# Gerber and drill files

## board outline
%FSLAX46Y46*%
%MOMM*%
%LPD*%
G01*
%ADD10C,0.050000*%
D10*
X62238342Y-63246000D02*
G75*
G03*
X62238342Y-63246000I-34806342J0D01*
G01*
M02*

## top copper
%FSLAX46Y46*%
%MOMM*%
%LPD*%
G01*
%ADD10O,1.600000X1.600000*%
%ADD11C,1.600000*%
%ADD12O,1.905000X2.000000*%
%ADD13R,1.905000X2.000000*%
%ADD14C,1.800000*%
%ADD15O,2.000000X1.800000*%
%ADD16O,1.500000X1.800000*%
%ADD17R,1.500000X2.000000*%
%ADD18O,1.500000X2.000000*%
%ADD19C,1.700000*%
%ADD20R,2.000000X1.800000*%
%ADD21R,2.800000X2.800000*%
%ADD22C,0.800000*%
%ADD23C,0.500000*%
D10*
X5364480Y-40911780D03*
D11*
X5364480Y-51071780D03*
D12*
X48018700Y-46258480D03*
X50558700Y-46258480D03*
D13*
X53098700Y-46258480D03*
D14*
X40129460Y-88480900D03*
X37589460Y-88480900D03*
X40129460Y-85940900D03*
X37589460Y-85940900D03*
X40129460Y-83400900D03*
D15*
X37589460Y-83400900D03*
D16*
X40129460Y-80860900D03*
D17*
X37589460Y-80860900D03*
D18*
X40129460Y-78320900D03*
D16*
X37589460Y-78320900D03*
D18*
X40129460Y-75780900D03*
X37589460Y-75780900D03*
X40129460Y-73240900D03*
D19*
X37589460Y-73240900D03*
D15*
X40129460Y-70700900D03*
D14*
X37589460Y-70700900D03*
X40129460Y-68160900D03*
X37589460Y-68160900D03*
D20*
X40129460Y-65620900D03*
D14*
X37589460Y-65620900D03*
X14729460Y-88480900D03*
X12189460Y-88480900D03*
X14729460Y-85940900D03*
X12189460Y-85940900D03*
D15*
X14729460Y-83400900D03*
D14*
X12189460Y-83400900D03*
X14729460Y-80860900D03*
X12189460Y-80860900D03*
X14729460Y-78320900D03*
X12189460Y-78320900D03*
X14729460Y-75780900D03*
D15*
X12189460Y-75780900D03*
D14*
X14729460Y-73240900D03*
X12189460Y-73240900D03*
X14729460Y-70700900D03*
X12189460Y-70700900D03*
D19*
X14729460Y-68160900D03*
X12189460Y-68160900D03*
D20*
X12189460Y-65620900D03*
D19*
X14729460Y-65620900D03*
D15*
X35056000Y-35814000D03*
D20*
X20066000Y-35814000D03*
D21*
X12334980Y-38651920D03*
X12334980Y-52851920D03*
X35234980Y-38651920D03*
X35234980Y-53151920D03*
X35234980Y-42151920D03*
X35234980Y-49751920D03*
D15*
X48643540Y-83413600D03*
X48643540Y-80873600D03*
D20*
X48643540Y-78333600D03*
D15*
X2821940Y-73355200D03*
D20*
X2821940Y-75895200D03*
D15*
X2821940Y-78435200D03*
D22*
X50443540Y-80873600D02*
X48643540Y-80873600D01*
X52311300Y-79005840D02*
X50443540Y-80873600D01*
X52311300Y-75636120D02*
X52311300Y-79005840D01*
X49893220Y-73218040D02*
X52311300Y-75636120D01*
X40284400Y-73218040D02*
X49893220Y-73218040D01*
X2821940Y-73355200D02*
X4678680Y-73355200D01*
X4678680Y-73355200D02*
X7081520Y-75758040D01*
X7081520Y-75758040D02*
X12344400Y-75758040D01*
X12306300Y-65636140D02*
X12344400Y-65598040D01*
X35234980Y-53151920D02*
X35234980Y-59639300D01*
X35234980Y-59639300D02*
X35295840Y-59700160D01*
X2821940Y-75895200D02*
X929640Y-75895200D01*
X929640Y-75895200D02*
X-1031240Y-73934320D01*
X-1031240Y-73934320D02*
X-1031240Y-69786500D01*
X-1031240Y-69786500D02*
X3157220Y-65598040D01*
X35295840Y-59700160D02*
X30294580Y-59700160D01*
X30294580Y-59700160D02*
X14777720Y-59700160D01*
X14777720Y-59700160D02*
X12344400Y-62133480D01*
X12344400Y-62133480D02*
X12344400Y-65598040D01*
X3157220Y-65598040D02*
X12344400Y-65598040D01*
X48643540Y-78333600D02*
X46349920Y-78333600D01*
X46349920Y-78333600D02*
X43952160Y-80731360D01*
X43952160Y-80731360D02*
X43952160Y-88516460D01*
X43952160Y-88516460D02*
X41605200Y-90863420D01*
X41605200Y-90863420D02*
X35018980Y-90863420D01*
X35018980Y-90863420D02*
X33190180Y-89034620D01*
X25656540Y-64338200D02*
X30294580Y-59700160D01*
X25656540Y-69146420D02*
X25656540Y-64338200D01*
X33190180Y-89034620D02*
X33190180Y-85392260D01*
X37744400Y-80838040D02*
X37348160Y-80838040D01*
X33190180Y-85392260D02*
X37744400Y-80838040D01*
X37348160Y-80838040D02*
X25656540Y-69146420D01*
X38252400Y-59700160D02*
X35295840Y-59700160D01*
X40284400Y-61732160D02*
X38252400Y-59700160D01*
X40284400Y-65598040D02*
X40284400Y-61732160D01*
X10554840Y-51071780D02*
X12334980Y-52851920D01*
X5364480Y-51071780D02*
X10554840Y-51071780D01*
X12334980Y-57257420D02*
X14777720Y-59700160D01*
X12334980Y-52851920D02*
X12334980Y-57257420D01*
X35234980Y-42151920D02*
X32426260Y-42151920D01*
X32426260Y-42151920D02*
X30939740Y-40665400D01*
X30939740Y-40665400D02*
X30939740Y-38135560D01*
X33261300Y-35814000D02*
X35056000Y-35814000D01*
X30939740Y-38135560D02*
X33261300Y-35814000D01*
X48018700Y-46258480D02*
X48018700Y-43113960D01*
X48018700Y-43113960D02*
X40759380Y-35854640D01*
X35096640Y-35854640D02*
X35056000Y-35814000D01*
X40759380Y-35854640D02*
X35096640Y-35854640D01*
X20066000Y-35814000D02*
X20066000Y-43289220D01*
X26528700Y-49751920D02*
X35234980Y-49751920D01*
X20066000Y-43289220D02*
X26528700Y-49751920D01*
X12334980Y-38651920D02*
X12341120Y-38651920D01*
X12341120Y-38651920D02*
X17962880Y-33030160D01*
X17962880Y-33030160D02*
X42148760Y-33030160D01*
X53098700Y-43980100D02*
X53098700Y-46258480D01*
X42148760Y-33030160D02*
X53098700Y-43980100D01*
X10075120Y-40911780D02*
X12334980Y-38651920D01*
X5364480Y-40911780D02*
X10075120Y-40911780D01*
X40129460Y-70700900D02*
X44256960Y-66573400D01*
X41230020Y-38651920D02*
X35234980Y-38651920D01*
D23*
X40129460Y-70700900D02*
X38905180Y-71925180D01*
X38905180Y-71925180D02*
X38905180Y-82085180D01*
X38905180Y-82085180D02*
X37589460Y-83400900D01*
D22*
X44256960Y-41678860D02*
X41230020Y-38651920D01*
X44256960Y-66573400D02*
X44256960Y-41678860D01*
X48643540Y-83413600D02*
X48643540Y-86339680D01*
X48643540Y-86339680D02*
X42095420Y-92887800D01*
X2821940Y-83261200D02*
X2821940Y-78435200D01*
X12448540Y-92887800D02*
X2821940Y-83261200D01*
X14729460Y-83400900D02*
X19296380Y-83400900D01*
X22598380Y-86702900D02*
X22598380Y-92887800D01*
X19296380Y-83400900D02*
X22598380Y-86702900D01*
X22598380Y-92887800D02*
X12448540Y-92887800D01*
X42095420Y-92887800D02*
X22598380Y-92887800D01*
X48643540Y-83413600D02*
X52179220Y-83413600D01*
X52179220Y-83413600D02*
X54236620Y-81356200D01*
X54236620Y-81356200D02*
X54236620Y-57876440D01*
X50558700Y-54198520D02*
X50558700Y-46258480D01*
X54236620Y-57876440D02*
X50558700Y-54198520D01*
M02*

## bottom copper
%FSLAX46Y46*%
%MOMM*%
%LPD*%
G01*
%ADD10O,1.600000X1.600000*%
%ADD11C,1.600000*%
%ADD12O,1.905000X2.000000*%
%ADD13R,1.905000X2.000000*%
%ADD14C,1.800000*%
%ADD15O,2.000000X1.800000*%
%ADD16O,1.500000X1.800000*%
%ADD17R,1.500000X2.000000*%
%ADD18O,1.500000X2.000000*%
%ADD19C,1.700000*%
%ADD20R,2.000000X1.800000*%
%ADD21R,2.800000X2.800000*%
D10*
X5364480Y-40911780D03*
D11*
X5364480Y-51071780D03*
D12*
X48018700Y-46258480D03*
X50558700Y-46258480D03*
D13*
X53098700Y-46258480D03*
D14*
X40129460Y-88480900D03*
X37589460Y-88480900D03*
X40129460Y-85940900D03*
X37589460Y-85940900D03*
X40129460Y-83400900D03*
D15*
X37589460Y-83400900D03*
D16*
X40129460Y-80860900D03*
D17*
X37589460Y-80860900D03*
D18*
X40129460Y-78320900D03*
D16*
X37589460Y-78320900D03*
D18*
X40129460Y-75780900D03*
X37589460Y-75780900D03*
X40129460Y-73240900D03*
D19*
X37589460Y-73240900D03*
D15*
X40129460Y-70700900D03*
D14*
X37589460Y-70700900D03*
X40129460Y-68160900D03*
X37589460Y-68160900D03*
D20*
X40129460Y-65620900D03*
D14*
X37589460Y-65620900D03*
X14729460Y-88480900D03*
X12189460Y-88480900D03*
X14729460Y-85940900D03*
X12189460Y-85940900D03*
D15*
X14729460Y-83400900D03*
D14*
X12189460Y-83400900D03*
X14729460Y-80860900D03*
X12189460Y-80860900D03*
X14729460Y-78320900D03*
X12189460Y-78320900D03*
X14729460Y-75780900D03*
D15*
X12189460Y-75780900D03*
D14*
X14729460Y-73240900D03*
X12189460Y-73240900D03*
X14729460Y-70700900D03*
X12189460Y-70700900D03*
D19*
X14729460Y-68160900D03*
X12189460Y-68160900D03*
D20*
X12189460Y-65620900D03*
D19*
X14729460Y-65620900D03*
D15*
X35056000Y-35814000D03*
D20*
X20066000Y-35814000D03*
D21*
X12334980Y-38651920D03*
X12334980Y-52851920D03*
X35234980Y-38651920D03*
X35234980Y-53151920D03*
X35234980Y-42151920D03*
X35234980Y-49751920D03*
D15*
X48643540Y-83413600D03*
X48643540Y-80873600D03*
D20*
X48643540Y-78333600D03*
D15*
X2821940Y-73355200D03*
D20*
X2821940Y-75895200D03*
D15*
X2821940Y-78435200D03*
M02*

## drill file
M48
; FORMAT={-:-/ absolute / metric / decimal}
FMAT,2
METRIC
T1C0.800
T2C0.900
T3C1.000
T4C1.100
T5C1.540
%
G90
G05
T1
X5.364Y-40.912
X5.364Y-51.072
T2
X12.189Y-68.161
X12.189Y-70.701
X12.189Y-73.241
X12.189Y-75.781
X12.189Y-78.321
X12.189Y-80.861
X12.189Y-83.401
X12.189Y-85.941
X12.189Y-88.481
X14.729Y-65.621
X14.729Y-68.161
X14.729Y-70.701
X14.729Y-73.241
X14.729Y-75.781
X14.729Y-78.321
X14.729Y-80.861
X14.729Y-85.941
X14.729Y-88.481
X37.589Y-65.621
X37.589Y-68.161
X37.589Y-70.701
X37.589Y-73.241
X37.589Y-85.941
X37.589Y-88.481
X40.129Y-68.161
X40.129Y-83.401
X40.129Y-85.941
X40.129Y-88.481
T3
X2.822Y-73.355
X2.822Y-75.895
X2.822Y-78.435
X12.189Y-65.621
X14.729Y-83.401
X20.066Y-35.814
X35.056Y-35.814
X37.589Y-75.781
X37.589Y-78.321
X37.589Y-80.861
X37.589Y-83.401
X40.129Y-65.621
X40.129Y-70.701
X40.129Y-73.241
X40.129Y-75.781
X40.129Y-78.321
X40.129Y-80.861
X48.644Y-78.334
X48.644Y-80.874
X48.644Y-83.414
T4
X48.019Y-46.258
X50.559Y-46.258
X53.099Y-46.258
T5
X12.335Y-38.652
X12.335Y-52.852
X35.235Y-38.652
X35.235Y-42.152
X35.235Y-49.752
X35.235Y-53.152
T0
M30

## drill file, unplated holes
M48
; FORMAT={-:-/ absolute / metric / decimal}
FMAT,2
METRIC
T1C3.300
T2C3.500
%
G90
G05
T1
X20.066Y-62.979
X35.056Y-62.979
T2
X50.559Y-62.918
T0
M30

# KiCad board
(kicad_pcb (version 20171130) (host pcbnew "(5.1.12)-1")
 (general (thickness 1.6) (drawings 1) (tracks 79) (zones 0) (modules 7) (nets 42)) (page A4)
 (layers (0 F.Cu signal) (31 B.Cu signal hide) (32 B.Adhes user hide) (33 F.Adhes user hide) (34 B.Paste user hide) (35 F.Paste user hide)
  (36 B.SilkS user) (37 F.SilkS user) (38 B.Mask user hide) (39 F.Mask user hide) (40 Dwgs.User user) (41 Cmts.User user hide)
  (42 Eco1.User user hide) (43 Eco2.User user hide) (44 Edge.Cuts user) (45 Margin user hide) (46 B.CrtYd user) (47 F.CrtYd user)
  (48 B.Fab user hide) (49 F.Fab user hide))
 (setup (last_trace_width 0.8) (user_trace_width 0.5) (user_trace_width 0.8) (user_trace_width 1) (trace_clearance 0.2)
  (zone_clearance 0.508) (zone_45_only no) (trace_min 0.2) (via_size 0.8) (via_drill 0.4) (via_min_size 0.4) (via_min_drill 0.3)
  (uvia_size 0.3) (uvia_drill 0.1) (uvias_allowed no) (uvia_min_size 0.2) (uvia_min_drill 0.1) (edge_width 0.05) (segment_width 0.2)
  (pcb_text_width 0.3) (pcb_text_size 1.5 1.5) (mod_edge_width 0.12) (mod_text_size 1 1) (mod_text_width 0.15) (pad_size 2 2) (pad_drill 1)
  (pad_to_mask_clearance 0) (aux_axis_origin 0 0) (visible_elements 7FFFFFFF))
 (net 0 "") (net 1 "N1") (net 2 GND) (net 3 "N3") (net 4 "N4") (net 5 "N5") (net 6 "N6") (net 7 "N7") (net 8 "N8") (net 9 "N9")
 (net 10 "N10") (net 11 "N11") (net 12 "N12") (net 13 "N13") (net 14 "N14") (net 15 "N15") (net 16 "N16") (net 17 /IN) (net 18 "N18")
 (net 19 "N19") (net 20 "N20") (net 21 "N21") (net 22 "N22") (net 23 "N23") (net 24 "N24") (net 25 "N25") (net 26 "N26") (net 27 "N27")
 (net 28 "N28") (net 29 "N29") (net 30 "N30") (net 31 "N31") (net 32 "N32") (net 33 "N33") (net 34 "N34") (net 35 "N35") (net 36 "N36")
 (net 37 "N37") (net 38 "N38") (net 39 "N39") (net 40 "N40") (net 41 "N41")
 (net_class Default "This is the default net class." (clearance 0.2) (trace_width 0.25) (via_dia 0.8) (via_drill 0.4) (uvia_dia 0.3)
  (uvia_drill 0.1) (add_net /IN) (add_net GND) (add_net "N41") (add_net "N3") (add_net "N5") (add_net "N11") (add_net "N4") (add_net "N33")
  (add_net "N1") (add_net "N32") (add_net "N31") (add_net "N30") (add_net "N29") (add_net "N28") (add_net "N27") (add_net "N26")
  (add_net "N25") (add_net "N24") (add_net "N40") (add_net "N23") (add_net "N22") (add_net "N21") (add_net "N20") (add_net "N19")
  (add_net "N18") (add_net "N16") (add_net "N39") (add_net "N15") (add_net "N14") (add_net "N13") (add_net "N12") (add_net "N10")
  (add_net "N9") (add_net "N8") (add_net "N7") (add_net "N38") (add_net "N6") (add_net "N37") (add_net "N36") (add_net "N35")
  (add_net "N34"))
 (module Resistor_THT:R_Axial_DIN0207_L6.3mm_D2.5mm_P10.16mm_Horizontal (layer F.Cu) (at 5.36448 51.07178 90)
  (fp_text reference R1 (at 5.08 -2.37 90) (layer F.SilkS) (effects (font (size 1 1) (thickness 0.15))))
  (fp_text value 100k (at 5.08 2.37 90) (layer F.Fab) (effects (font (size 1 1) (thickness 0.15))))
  (pad 2 thru_hole oval (at 10.16 0 90) (size 1.6 1.6) (drill 0.8) (layers *.Cu *.Mask) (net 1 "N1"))
  (pad 1 thru_hole circle (at 0 0 90) (size 1.6 1.6) (drill 0.8) (layers *.Cu *.Mask) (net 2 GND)))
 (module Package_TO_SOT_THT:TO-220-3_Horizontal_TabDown (layer F.Cu) (at 53.0987 46.25848 180)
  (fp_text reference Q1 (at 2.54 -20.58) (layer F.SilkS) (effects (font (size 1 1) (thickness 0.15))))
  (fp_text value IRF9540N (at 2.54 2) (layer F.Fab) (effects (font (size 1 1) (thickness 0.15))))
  (pad 3 thru_hole oval (at 5.08 0 180) (size 1.905 2) (drill 1.1) (layers *.Cu *.Mask) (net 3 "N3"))
  (pad 2 thru_hole oval (at 2.54 0 180) (size 1.905 2) (drill 1.1) (layers *.Cu *.Mask) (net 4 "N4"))
  (pad 1 thru_hole rect (at 0 0 180) (size 1.905 2) (drill 1.1) (layers *.Cu *.Mask) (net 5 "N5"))
  (pad "" np_thru_hole oval (at 2.54 -16.66 180) (size 3.5 3.5) (drill 3.5) (layers *.Cu *.Mask)))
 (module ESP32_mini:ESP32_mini (layer F.Cu) (at 26.15946 77.0509)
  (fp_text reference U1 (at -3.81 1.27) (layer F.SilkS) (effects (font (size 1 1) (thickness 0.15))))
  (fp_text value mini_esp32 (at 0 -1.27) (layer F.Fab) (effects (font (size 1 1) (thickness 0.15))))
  (pad 40 thru_hole circle (at 13.97 11.43 270) (size 1.8 1.8) (drill 0.9) (layers *.Cu *.Mask) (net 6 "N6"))
  (pad 39 thru_hole circle (at 11.43 11.43 270) (size 1.8 1.8) (drill 0.9) (layers *.Cu *.Mask) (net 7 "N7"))
  (pad 38 thru_hole circle (at 13.97 8.89 270) (size 1.8 1.8) (drill 0.9) (layers *.Cu *.Mask) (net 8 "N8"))
  (pad 37 thru_hole circle (at 11.43 8.89 270) (size 1.8 1.8) (drill 0.9) (layers *.Cu *.Mask) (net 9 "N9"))
  (pad 36 thru_hole circle (at 13.97 6.35 270) (size 1.8 1.8) (drill 0.9) (layers *.Cu *.Mask) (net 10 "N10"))
  (pad 35 thru_hole oval (at 11.43 6.35) (size 2 1.8) (drill 1) (layers *.Cu *.Mask) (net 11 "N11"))
  (pad 34 thru_hole oval (at 13.97 3.81) (size 1.5 1.8) (drill 1) (layers *.Cu *.Mask) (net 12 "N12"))
  (pad 33 thru_hole rect (at 11.43 3.81) (size 1.5 2) (drill 1) (layers *.Cu *.Mask) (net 2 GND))
  (pad 32 thru_hole oval (at 13.97 1.27) (size 1.5 2) (drill 1) (layers *.Cu *.Mask) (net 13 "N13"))
  (pad 31 thru_hole oval (at 11.43 1.27) (size 1.5 1.8) (drill 1) (layers *.Cu *.Mask) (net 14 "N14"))
  (pad 30 thru_hole oval (at 13.97 -1.27) (size 1.5 2) (drill 1) (layers *.Cu *.Mask) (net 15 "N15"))
  (pad 29 thru_hole oval (at 11.43 -1.27) (size 1.5 2) (drill 1) (layers *.Cu *.Mask) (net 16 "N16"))
  (pad 28 thru_hole oval (at 13.97 -3.81) (size 1.5 2) (drill 1) (layers *.Cu *.Mask) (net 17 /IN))
  (pad 27 thru_hole circle (at 11.43 -3.81 270) (size 1.7 1.7) (drill 0.9) (layers *.Cu *.Mask) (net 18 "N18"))
  (pad 26 thru_hole oval (at 13.97 -6.35) (size 2 1.8) (drill 1) (layers *.Cu *.Mask) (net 11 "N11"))
  (pad 25 thru_hole circle (at 11.43 -6.35 270) (size 1.8 1.8) (drill 0.9) (layers *.Cu *.Mask) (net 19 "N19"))
  (pad 24 thru_hole circle (at 13.97 -8.89 270) (size 1.8 1.8) (drill 0.9) (layers *.Cu *.Mask) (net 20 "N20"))
  (pad 23 thru_hole circle (at 11.43 -8.89 270) (size 1.8 1.8) (drill 0.9) (layers *.Cu *.Mask) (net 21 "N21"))
  (pad 22 thru_hole rect (at 13.97 -11.43) (size 2 1.8) (drill 1) (layers *.Cu *.Mask) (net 2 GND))
  (pad 21 thru_hole circle (at 11.43 -11.43 270) (size 1.8 1.8) (drill 0.9) (layers *.Cu *.Mask) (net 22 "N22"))
  (pad 20 thru_hole circle (at -11.43 11.43 270) (size 1.8 1.8) (drill 0.9) (layers *.Cu *.Mask) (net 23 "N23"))
  (pad 19 thru_hole circle (at -13.97 11.43 270) (size 1.8 1.8) (drill 0.9) (layers *.Cu *.Mask) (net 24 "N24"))
  (pad 18 thru_hole circle (at -11.43 8.89 270) (size 1.8 1.8) (drill 0.9) (layers *.Cu *.Mask) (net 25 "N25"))
  (pad 17 thru_hole circle (at -13.97 8.89 270) (size 1.8 1.8) (drill 0.9) (layers *.Cu *.Mask) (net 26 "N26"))
  (pad 16 thru_hole oval (at -11.43 6.35) (size 2 1.8) (drill 1) (layers *.Cu *.Mask) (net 4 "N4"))
  (pad 15 thru_hole circle (at -13.97 6.35 270) (size 1.8 1.8) (drill 0.9) (layers *.Cu *.Mask) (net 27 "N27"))
  (pad 14 thru_hole circle (at -11.43 3.81 270) (size 1.8 1.8) (drill 0.9) (layers *.Cu *.Mask) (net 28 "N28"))
  (pad 13 thru_hole circle (at -13.97 3.81 270) (size 1.8 1.8) (drill 0.9) (layers *.Cu *.Mask) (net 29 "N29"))
  (pad 12 thru_hole circle (at -11.43 1.27 270) (size 1.8 1.8) (drill 0.9) (layers *.Cu *.Mask) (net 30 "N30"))
  (pad 11 thru_hole circle (at -13.97 1.27 270) (size 1.8 1.8) (drill 0.9) (layers *.Cu *.Mask) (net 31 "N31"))
  (pad 10 thru_hole circle (at -11.43 -1.27 270) (size 1.8 1.8) (drill 0.9) (layers *.Cu *.Mask) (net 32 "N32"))
  (pad 9 thru_hole oval (at -13.97 -1.27) (size 2 1.8) (drill 0.9) (layers *.Cu *.Mask) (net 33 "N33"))
  (pad 8 thru_hole circle (at -11.43 -3.81 270) (size 1.8 1.8) (drill 0.9) (layers *.Cu *.Mask) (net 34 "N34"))
  (pad 7 thru_hole circle (at -13.97 -3.81 270) (size 1.8 1.8) (drill 0.9) (layers *.Cu *.Mask) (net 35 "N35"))
  (pad 6 thru_hole circle (at -11.43 -6.35 270) (size 1.8 1.8) (drill 0.9) (layers *.Cu *.Mask) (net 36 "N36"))
  (pad 5 thru_hole circle (at -13.97 -6.35 270) (size 1.8 1.8) (drill 0.9) (layers *.Cu *.Mask) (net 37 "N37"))
  (pad 4 thru_hole circle (at -11.43 -8.89 270) (size 1.7 1.7) (drill 0.9) (layers *.Cu *.Mask) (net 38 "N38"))
  (pad 3 thru_hole circle (at -13.97 -8.89 270) (size 1.7 1.7) (drill 0.9) (layers *.Cu *.Mask) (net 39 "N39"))
  (pad 1 thru_hole rect (at -13.97 -11.43) (size 2 1.8) (drill 1) (layers *.Cu *.Mask) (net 2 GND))
  (pad 2 thru_hole circle (at -11.43 -11.43 270) (size 1.7 1.7) (drill 0.9) (layers *.Cu *.Mask) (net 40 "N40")))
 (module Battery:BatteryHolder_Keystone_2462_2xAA (layer B.Cu) (at 20.066 35.814 270)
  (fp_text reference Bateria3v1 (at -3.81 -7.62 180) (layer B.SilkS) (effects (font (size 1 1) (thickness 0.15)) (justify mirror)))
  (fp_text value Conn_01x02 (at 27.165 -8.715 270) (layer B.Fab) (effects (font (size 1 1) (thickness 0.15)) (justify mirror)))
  (pad "" np_thru_hole circle (at 27.165 0 270) (size 3.3 3.3) (drill 3.3) (layers *.Cu *.Mask))
  (pad "" np_thru_hole circle (at 27.165 -14.99 270) (size 3.3 3.3) (drill 3.3) (layers *.Cu *.Mask))
  (pad 2 thru_hole oval (at 0 -14.99 270) (size 1.8 2) (drill 1) (layers *.Cu *.Mask) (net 3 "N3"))
  (pad 1 thru_hole rect (at 0 0 270) (size 1.8 2) (drill 1) (layers *.Cu *.Mask) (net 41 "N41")))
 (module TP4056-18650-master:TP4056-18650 (layer F.Cu) (at 10.63498 36.95192)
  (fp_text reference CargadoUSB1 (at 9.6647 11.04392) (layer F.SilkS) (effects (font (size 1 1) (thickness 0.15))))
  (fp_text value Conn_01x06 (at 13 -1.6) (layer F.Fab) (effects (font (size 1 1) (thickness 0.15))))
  (pad 1 thru_hole rect (at 1.7 1.7) (size 2.8 2.8) (drill 1.54) (layers *.Cu *.Mask) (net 5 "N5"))
  (pad 2 thru_hole rect (at 1.7 15.9) (size 2.8 2.8) (drill 1.54) (layers *.Cu *.Mask) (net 2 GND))
  (pad 3 thru_hole rect (at 24.6 1.7) (size 2.8 2.8) (drill 1.54) (layers *.Cu *.Mask) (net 11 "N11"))
  (pad 4 thru_hole rect (at 24.6 16.2) (size 2.8 2.8) (drill 1.54) (layers *.Cu *.Mask) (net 2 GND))
  (pad 5 thru_hole rect (at 24.6 5.2) (size 2.8 2.8) (drill 1.54) (layers *.Cu *.Mask) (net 3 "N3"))
  (pad 6 thru_hole rect (at 24.6 12.8) (size 2.8 2.8) (drill 1.54) (layers *.Cu *.Mask) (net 41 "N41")))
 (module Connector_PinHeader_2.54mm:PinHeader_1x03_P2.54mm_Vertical (layer F.Cu) (at 48.64354 78.3336)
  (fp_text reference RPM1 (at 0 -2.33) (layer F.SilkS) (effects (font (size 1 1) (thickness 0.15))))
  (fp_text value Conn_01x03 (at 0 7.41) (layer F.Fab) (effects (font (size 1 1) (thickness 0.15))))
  (pad 3 thru_hole oval (at 0 5.08) (size 2 1.8) (drill 1) (layers *.Cu *.Mask) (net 4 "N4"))
  (pad 2 thru_hole oval (at 0 2.54) (size 2 1.8) (drill 1) (layers *.Cu *.Mask) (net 17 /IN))
  (pad 1 thru_hole rect (at 0 0) (size 2 1.8) (drill 1) (layers *.Cu *.Mask) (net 2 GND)))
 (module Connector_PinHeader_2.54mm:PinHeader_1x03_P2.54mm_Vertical (layer F.Cu) (at 2.82194 78.4352 180)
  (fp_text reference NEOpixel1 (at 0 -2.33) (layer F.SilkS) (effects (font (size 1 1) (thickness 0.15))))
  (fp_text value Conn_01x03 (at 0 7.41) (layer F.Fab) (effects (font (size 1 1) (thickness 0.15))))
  (pad 3 thru_hole oval (at 0 5.08 180) (size 2 1.8) (drill 1) (layers *.Cu *.Mask) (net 33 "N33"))
  (pad 2 thru_hole rect (at 0 2.54 180) (size 2 1.8) (drill 1) (layers *.Cu *.Mask) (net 2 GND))
  (pad 1 thru_hole oval (at 0 0 180) (size 2 1.8) (drill 1) (layers *.Cu *.Mask) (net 4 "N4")))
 (gr_circle (center 27.432 63.246) (end 28.194 98.044) (layer Edge.Cuts) (width 0.05))
 (segment (start 50.44354 80.8736) (end 48.64354 80.8736) (width 0.8) (layer F.Cu) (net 17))
 (segment (start 52.3113 79.00584) (end 50.44354 80.8736) (width 0.8) (layer F.Cu) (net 17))
 (segment (start 52.3113 75.63612) (end 52.3113 79.00584) (width 0.8) (layer F.Cu) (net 17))
 (segment (start 49.89322 73.21804) (end 52.3113 75.63612) (width 0.8) (layer F.Cu) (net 17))
 (segment (start 40.2844 73.21804) (end 49.89322 73.21804) (width 0.8) (layer F.Cu) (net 17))
 (segment (start 2.82194 73.3552) (end 4.67868 73.3552) (width 0.8) (layer F.Cu) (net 33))
 (segment (start 4.67868 73.3552) (end 7.08152 75.75804) (width 0.8) (layer F.Cu) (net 33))
 (segment (start 7.08152 75.75804) (end 12.3444 75.75804) (width 0.8) (layer F.Cu) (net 33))
 (segment (start 12.3063 65.63614) (end 12.3444 65.59804) (width 0.8) (layer F.Cu) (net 2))
 (segment (start 35.23498 53.15192) (end 35.23498 59.6393) (width 0.8) (layer F.Cu) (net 2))
 (segment (start 35.23498 59.6393) (end 35.29584 59.70016) (width 0.8) (layer F.Cu) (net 2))
 (segment (start 2.82194 75.8952) (end 0.92964 75.8952) (width 0.8) (layer F.Cu) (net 2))
 (segment (start 0.92964 75.8952) (end -1.03124 73.93432) (width 0.8) (layer F.Cu) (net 2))
 (segment (start -1.03124 73.93432) (end -1.03124 69.7865) (width 0.8) (layer F.Cu) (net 2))
 (segment (start -1.03124 69.7865) (end 3.15722 65.59804) (width 0.8) (layer F.Cu) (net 2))
 (segment (start 35.29584 59.70016) (end 30.29458 59.70016) (width 0.8) (layer F.Cu) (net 2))
 (segment (start 30.29458 59.70016) (end 14.77772 59.70016) (width 0.8) (layer F.Cu) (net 2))
 (segment (start 14.77772 59.70016) (end 12.3444 62.13348) (width 0.8) (layer F.Cu) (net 2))
 (segment (start 12.3444 62.13348) (end 12.3444 65.59804) (width 0.8) (layer F.Cu) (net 2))
 (segment (start 3.15722 65.59804) (end 12.3444 65.59804) (width 0.8) (layer F.Cu) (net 2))
 (segment (start 48.64354 78.3336) (end 46.34992 78.3336) (width 0.8) (layer F.Cu) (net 2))
 (segment (start 46.34992 78.3336) (end 43.95216 80.73136) (width 0.8) (layer F.Cu) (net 2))
 (segment (start 43.95216 80.73136) (end 43.95216 88.51646) (width 0.8) (layer F.Cu) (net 2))
 (segment (start 43.95216 88.51646) (end 41.6052 90.86342) (width 0.8) (layer F.Cu) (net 2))
 (segment (start 41.6052 90.86342) (end 35.01898 90.86342) (width 0.8) (layer F.Cu) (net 2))
 (segment (start 35.01898 90.86342) (end 33.19018 89.03462) (width 0.8) (layer F.Cu) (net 2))
 (segment (start 25.65654 64.3382) (end 30.29458 59.70016) (width 0.8) (layer F.Cu) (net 2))
 (segment (start 25.65654 69.14642) (end 25.65654 64.3382) (width 0.8) (layer F.Cu) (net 2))
 (segment (start 33.19018 89.03462) (end 33.19018 85.39226) (width 0.8) (layer F.Cu) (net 2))
 (segment (start 37.7444 80.83804) (end 37.34816 80.83804) (width 0.8) (layer F.Cu) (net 2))
 (segment (start 33.19018 85.39226) (end 37.7444 80.83804) (width 0.8) (layer F.Cu) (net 2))
 (segment (start 37.34816 80.83804) (end 25.65654 69.14642) (width 0.8) (layer F.Cu) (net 2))
 (segment (start 38.2524 59.70016) (end 35.29584 59.70016) (width 0.8) (layer F.Cu) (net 2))
 (segment (start 40.2844 61.73216) (end 38.2524 59.70016) (width 0.8) (layer F.Cu) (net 2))
 (segment (start 40.2844 65.59804) (end 40.2844 61.73216) (width 0.8) (layer F.Cu) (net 2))
 (segment (start 10.55484 51.07178) (end 12.33498 52.85192) (width 0.8) (layer F.Cu) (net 2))
 (segment (start 5.36448 51.07178) (end 10.55484 51.07178) (width 0.8) (layer F.Cu) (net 2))
 (segment (start 12.33498 57.25742) (end 14.77772 59.70016) (width 0.8) (layer F.Cu) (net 2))
 (segment (start 12.33498 52.85192) (end 12.33498 57.25742) (width 0.8) (layer F.Cu) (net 2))
 (segment (start 35.23498 42.15192) (end 32.42626 42.15192) (width 0.8) (layer F.Cu) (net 3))
 (segment (start 32.42626 42.15192) (end 30.93974 40.6654) (width 0.8) (layer F.Cu) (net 3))
 (segment (start 30.93974 40.6654) (end 30.93974 38.13556) (width 0.8) (layer F.Cu) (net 3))
 (segment (start 33.2613 35.814) (end 35.056 35.814) (width 0.8) (layer F.Cu) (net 3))
 (segment (start 30.93974 38.13556) (end 33.2613 35.814) (width 0.8) (layer F.Cu) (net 3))
 (segment (start 48.0187 46.25848) (end 48.0187 43.11396) (width 0.8) (layer F.Cu) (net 3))
 (segment (start 48.0187 43.11396) (end 40.75938 35.85464) (width 0.8) (layer F.Cu) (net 3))
 (segment (start 35.09664 35.85464) (end 35.056 35.814) (width 0.8) (layer F.Cu) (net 3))
 (segment (start 40.75938 35.85464) (end 35.09664 35.85464) (width 0.8) (layer F.Cu) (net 3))
 (segment (start 20.066 35.814) (end 20.066 43.28922) (width 0.8) (layer F.Cu) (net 41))
 (segment (start 26.5287 49.75192) (end 35.23498 49.75192) (width 0.8) (layer F.Cu) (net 41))
 (segment (start 20.066 43.28922) (end 26.5287 49.75192) (width 0.8) (layer F.Cu) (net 41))
 (segment (start 12.33498 38.65192) (end 12.34112 38.65192) (width 0.8) (layer F.Cu) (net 5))
 (segment (start 12.34112 38.65192) (end 17.96288 33.03016) (width 0.8) (layer F.Cu) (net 5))
 (segment (start 17.96288 33.03016) (end 42.14876 33.03016) (width 0.8) (layer F.Cu) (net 5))
 (segment (start 53.0987 43.9801) (end 53.0987 46.25848) (width 0.8) (layer F.Cu) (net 5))
 (segment (start 42.14876 33.03016) (end 53.0987 43.9801) (width 0.8) (layer F.Cu) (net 5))
 (segment (start 10.07512 40.91178) (end 12.33498 38.65192) (width 0.8) (layer F.Cu) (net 5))
 (segment (start 5.36448 40.91178) (end 10.07512 40.91178) (width 0.8) (layer F.Cu) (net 5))
 (segment (start 40.12946 70.7009) (end 44.25696 66.5734) (width 0.8) (layer F.Cu) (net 11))
 (segment (start 41.23002 38.65192) (end 35.23498 38.65192) (width 0.8) (layer F.Cu) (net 11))
 (segment (start 40.12946 70.7009) (end 38.90518 71.92518) (width 0.5) (layer F.Cu) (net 11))
 (segment (start 38.90518 71.92518) (end 38.90518 82.08518) (width 0.5) (layer F.Cu) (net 11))
 (segment (start 38.90518 82.08518) (end 37.58946 83.4009) (width 0.5) (layer F.Cu) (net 11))
 (segment (start 44.25696 41.67886) (end 41.23002 38.65192) (width 0.8) (layer F.Cu) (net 11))
 (segment (start 44.25696 66.5734) (end 44.25696 41.67886) (width 0.8) (layer F.Cu) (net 11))
 (segment (start 48.64354 83.4136) (end 48.64354 86.33968) (width 0.8) (layer F.Cu) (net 4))
 (segment (start 48.64354 86.33968) (end 42.09542 92.8878) (width 0.8) (layer F.Cu) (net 4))
 (segment (start 2.82194 83.2612) (end 2.82194 78.4352) (width 0.8) (layer F.Cu) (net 4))
 (segment (start 12.44854 92.8878) (end 2.82194 83.2612) (width 0.8) (layer F.Cu) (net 4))
 (segment (start 14.72946 83.4009) (end 19.29638 83.4009) (width 0.8) (layer F.Cu) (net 4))
 (segment (start 22.59838 86.7029) (end 22.59838 92.8878) (width 0.8) (layer F.Cu) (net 4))
 (segment (start 19.29638 83.4009) (end 22.59838 86.7029) (width 0.8) (layer F.Cu) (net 4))
 (segment (start 22.59838 92.8878) (end 12.44854 92.8878) (width 0.8) (layer F.Cu) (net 4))
 (segment (start 42.09542 92.8878) (end 22.59838 92.8878) (width 0.8) (layer F.Cu) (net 4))
 (segment (start 48.64354 83.4136) (end 52.17922 83.4136) (width 0.8) (layer F.Cu) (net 4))
 (segment (start 52.17922 83.4136) (end 54.23662 81.3562) (width 0.8) (layer F.Cu) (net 4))
 (segment (start 54.23662 81.3562) (end 54.23662 57.87644) (width 0.8) (layer F.Cu) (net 4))
 (segment (start 50.5587 54.19852) (end 50.5587 46.25848) (width 0.8) (layer F.Cu) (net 4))
 (segment (start 54.23662 57.87644) (end 50.5587 54.19852) (width 0.8) (layer F.Cu) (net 4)))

